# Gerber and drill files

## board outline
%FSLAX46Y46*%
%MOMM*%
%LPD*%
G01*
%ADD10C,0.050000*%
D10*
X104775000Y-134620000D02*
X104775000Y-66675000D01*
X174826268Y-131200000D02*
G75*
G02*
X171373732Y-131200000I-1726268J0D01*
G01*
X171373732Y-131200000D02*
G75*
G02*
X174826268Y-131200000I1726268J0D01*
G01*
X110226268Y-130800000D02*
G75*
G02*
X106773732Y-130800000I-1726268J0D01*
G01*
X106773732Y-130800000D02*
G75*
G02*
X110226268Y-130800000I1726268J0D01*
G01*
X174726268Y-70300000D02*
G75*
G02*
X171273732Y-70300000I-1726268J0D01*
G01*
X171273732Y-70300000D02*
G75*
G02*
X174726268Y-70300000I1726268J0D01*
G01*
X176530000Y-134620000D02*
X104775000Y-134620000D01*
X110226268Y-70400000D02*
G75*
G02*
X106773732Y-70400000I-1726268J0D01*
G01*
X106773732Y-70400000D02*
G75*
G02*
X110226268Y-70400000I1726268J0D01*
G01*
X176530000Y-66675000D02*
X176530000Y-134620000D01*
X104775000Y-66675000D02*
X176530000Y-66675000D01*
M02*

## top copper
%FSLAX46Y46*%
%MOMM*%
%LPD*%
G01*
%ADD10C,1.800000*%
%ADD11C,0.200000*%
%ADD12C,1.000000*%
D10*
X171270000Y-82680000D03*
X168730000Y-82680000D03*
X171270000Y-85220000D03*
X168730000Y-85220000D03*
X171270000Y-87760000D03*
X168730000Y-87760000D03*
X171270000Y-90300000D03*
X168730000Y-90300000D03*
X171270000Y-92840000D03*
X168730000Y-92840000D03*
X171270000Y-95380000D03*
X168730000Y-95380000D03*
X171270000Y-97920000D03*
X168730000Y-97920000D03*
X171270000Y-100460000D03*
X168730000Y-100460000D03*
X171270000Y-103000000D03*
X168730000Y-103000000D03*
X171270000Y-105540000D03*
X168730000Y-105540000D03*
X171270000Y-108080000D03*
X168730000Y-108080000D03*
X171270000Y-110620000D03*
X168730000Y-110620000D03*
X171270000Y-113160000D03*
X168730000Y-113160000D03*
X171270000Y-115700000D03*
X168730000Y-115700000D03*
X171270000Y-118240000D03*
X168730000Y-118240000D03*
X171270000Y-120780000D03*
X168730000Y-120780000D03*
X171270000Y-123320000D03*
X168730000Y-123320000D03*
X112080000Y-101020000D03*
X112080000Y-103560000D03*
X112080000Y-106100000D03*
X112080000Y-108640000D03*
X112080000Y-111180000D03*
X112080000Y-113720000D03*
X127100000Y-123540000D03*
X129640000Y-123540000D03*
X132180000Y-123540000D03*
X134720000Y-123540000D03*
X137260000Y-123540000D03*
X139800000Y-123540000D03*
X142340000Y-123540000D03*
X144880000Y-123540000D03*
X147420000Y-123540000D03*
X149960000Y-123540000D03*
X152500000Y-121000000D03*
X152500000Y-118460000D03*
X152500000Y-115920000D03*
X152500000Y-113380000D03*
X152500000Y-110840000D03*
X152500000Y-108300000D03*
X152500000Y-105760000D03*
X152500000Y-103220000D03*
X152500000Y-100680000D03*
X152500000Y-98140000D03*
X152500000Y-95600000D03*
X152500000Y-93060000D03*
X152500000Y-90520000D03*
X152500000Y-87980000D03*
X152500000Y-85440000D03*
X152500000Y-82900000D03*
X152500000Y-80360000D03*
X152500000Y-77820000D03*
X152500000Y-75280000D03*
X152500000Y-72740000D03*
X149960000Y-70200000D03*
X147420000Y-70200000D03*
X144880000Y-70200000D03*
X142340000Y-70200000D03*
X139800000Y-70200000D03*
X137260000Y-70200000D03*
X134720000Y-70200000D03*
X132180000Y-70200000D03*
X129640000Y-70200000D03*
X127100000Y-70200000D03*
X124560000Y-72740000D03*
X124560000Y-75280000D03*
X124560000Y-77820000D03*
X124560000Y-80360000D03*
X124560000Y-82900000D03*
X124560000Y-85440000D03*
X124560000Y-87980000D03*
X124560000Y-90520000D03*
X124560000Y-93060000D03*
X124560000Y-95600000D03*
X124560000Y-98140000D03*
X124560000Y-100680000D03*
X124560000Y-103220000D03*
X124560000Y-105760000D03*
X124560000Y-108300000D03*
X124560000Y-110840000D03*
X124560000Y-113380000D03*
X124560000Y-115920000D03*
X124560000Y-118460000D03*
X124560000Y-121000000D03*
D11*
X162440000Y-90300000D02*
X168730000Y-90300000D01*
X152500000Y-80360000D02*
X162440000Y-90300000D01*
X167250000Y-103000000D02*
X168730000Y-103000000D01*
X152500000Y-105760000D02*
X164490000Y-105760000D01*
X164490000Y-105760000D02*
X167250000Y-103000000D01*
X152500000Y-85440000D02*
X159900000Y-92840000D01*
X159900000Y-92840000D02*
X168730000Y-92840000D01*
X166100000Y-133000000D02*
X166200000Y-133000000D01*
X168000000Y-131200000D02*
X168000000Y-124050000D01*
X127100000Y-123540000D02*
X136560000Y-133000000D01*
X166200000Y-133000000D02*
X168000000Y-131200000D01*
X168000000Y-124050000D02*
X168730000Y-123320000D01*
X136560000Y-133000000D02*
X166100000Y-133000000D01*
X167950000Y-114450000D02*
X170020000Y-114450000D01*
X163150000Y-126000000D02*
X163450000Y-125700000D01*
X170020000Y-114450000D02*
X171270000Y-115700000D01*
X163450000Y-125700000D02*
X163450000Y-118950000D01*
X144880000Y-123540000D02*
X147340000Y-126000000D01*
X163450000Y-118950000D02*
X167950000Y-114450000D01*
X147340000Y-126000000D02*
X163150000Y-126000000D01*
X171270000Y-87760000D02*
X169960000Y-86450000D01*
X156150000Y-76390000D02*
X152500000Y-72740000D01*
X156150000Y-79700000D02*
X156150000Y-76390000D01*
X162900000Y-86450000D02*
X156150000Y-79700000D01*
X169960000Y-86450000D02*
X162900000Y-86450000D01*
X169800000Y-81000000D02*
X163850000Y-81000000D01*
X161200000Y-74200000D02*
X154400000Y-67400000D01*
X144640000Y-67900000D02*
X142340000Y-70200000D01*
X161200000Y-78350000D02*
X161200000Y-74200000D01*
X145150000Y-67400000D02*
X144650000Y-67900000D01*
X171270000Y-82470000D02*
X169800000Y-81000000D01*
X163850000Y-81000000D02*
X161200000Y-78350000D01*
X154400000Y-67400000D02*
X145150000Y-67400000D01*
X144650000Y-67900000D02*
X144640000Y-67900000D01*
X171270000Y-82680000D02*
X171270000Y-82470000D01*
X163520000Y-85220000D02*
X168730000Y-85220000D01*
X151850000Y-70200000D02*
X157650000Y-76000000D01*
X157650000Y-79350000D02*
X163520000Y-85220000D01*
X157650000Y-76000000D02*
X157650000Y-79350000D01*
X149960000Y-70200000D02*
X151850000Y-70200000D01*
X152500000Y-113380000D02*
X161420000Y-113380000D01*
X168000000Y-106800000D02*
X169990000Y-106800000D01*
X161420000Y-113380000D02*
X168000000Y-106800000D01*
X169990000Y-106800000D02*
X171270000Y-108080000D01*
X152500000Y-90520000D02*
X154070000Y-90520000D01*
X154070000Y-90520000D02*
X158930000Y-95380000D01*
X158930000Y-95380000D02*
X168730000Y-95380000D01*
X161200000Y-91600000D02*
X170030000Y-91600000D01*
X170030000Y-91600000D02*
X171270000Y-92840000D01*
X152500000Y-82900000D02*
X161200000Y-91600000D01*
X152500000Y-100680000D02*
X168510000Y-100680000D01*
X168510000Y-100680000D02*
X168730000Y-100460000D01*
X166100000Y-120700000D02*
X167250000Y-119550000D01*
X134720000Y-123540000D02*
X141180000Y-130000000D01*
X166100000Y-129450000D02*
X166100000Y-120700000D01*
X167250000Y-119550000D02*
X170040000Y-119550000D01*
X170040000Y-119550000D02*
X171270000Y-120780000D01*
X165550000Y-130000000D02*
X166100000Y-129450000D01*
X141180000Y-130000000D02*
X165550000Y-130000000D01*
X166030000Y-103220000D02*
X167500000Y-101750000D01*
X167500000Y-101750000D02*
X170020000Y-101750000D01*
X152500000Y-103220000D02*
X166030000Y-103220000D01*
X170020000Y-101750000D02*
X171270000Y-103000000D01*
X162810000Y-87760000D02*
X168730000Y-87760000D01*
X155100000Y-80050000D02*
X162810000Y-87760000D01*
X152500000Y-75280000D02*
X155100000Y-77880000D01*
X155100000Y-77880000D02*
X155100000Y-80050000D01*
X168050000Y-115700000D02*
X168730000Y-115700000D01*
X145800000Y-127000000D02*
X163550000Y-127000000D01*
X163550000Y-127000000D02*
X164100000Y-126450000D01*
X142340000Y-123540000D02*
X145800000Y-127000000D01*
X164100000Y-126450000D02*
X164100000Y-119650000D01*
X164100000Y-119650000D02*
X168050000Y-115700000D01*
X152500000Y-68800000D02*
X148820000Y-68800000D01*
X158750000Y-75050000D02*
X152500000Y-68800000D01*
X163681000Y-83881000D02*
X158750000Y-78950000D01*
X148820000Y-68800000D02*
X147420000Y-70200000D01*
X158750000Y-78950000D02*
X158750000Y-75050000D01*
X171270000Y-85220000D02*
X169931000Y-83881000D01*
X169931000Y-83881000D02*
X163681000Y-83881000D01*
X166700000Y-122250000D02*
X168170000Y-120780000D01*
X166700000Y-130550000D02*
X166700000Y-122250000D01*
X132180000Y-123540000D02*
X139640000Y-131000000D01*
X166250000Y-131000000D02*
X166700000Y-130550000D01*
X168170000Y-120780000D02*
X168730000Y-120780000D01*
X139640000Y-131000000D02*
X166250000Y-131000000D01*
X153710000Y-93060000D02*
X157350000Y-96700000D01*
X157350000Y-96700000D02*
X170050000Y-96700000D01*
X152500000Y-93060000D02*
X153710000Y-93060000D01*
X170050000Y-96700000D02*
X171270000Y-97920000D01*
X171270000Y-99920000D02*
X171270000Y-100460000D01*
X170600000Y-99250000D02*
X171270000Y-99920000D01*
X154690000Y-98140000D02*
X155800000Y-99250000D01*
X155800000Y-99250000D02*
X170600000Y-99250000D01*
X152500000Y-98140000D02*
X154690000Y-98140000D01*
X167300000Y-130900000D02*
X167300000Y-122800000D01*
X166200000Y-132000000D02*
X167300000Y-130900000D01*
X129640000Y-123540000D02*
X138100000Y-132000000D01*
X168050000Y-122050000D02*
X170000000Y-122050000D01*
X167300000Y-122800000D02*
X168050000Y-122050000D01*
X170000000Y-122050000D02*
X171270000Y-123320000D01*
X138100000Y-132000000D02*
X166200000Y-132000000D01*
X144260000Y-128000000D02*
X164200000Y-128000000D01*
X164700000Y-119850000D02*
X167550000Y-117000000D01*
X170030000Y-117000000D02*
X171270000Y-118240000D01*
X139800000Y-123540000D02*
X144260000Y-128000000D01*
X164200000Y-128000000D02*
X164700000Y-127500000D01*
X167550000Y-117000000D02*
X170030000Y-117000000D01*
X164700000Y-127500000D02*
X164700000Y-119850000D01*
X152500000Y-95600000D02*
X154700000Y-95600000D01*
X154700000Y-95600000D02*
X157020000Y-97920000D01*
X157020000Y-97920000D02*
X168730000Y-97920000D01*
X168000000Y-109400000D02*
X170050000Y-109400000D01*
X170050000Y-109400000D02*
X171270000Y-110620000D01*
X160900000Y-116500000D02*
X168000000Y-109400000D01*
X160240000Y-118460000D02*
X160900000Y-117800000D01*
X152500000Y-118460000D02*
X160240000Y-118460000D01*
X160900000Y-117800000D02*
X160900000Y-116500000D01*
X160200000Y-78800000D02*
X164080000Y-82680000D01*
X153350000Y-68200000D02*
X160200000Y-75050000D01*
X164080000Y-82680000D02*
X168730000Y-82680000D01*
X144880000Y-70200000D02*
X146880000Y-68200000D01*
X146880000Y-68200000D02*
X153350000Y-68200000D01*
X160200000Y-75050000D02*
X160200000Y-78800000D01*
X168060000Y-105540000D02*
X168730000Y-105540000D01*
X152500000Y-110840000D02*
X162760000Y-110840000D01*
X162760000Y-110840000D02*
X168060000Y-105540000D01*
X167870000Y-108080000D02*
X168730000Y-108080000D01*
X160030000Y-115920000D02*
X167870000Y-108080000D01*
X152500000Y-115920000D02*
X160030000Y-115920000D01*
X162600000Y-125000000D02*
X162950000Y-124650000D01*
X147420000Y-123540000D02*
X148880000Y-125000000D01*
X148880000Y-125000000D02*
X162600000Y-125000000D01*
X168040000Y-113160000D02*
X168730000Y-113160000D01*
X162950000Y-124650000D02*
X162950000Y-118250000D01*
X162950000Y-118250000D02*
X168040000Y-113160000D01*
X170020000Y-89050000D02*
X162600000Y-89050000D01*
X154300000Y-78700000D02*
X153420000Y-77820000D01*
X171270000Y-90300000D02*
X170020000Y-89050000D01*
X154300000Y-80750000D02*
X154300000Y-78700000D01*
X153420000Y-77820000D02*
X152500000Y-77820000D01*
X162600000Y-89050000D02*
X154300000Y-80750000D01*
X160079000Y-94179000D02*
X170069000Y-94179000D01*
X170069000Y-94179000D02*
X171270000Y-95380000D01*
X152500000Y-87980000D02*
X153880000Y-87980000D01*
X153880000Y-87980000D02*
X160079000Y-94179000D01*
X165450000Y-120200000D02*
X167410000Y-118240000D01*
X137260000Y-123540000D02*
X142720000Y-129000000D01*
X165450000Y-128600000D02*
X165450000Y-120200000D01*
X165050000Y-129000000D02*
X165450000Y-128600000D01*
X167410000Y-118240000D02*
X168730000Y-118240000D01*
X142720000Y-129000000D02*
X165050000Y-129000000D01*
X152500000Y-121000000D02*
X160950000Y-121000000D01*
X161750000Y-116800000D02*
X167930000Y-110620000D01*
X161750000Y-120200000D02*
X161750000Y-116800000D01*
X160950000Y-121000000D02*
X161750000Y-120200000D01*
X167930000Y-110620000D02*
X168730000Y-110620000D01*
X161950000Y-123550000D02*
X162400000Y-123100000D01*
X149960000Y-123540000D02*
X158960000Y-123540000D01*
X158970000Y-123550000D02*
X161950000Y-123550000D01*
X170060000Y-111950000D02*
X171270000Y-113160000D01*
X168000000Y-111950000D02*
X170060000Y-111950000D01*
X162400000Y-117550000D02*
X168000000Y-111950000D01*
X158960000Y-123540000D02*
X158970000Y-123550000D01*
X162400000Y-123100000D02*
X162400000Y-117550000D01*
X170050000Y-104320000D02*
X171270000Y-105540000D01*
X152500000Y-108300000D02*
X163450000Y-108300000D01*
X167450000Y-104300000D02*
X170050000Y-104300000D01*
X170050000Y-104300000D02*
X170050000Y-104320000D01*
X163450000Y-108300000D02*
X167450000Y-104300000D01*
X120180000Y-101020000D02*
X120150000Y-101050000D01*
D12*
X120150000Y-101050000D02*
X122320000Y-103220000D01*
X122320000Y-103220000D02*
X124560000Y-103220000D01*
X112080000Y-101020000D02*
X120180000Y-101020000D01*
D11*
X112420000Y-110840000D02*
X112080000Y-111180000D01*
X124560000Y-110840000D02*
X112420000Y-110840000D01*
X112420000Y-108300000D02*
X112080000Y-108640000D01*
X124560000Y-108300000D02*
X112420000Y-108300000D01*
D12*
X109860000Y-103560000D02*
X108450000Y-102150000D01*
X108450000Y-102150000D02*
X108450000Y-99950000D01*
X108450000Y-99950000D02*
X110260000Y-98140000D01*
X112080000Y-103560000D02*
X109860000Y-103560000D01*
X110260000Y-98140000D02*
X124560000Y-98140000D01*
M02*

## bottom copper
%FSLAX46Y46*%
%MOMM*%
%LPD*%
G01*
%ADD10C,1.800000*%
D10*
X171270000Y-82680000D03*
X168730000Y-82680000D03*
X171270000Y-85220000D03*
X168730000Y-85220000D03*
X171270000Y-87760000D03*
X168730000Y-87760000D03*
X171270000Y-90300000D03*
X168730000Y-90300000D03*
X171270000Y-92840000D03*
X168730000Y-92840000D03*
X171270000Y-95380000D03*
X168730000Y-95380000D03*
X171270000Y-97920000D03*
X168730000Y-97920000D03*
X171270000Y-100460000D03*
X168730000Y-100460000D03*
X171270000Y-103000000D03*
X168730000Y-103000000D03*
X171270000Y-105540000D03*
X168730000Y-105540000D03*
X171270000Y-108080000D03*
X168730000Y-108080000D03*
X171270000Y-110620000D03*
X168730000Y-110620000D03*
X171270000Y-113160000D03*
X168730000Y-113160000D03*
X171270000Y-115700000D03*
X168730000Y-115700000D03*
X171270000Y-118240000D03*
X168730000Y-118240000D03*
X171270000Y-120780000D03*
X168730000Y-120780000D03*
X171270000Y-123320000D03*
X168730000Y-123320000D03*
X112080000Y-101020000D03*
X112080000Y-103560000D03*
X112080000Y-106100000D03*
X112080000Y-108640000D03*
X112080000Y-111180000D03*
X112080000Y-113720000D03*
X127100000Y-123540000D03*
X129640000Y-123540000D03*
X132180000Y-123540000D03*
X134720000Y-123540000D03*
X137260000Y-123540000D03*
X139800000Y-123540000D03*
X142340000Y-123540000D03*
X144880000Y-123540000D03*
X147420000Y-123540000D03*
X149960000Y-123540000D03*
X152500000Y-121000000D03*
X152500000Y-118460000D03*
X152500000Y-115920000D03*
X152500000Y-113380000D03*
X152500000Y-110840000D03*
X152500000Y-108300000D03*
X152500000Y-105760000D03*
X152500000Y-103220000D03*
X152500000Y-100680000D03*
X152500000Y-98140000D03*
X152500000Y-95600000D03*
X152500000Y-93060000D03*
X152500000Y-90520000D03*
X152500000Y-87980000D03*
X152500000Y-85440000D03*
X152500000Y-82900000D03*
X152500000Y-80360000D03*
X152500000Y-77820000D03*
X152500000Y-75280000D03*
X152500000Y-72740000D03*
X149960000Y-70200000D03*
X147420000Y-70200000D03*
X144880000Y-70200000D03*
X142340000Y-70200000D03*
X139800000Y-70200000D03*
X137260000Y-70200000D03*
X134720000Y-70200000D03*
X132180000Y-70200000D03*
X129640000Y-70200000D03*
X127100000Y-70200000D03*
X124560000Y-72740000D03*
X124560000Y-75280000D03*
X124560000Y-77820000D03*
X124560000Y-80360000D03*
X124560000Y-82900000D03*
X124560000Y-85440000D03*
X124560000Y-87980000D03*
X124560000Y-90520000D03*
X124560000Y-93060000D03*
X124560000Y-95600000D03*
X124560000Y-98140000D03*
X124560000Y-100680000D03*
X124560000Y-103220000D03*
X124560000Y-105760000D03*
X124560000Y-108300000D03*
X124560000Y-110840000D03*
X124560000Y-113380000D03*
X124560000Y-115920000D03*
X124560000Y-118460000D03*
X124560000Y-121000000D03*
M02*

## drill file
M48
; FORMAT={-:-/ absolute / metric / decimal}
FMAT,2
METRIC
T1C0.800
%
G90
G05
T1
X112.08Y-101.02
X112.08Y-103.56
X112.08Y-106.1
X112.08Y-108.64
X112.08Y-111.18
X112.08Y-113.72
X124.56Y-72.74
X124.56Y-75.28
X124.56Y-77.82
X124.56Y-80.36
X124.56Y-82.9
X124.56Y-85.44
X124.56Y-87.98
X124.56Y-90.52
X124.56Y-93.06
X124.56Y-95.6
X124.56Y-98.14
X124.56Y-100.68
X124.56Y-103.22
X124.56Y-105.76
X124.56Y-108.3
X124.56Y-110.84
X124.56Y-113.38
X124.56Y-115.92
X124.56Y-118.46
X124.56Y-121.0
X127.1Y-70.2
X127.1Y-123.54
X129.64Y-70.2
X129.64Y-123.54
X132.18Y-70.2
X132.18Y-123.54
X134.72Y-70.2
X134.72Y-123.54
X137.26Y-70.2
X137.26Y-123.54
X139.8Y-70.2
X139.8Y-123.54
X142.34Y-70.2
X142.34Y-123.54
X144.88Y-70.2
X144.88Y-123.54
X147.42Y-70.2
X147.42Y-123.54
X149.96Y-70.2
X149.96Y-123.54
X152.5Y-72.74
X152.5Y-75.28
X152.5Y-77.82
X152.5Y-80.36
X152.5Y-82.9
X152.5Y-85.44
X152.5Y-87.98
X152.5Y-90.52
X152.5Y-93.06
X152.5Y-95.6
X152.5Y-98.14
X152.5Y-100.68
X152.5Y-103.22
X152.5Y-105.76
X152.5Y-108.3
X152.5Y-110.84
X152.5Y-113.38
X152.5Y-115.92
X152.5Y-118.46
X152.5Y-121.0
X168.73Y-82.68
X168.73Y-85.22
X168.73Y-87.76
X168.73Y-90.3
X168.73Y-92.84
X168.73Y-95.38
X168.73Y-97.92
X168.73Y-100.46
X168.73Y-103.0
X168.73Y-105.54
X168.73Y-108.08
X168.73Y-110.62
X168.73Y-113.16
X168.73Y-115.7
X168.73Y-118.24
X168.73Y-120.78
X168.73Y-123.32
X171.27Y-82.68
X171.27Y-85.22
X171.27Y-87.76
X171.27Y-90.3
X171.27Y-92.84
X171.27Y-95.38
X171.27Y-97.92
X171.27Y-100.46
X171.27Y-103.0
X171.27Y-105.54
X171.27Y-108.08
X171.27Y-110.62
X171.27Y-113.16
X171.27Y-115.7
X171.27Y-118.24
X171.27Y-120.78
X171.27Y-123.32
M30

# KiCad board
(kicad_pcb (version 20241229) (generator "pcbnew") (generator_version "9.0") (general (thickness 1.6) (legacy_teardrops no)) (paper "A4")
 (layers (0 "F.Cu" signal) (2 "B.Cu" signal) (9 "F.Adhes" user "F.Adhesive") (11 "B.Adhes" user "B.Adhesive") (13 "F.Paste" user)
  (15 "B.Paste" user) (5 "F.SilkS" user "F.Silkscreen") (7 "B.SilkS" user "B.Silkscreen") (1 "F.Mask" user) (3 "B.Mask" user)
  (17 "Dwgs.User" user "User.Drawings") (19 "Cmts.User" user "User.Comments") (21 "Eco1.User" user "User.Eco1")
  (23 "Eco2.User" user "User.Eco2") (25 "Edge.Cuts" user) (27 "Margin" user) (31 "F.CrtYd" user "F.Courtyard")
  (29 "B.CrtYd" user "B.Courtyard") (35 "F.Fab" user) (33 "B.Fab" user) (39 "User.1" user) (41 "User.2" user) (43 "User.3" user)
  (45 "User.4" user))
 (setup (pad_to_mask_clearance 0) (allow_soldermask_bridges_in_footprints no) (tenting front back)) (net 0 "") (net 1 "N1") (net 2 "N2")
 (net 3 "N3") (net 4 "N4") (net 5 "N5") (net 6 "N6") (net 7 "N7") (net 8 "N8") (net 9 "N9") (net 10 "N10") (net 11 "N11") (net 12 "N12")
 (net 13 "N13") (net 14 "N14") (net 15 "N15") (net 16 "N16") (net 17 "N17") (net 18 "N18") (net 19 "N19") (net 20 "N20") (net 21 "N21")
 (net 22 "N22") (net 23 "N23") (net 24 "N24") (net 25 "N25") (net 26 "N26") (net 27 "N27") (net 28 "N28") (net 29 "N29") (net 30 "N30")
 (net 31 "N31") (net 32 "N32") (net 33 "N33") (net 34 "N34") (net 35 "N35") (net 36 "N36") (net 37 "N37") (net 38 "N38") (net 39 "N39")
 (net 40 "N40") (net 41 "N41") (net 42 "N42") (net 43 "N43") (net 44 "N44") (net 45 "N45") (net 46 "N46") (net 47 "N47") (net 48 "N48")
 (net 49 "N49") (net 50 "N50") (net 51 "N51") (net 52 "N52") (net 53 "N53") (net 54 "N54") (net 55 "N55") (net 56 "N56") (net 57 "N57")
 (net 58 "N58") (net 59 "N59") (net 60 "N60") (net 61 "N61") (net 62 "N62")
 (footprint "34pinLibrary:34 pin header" (layer "F.Cu") (at 168.73 82.68)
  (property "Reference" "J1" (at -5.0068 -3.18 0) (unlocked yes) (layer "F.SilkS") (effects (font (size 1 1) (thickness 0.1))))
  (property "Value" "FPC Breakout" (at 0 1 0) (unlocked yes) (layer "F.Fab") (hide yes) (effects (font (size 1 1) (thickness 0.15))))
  (pad "1" thru_hole circle (at 2.54 0) (size 1.8 1.8) (drill 0.8) (layers "*.Cu" "*.Mask") (remove_unused_layers no) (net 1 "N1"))
  (pad "2" thru_hole circle (at 0 0) (size 1.8 1.8) (drill 0.8) (layers "*.Cu" "*.Mask") (remove_unused_layers no) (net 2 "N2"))
  (pad "3" thru_hole circle (at 2.54 2.54) (size 1.8 1.8) (drill 0.8) (layers "*.Cu" "*.Mask") (remove_unused_layers no) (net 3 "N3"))
  (pad "4" thru_hole circle (at 0 2.54) (size 1.8 1.8) (drill 0.8) (layers "*.Cu" "*.Mask") (remove_unused_layers no) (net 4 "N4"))
  (pad "5" thru_hole circle (at 2.54 5.08) (size 1.8 1.8) (drill 0.8) (layers "*.Cu" "*.Mask") (remove_unused_layers no) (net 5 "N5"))
  (pad "6" thru_hole circle (at 0 5.08) (size 1.8 1.8) (drill 0.8) (layers "*.Cu" "*.Mask") (remove_unused_layers no) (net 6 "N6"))
  (pad "7" thru_hole circle (at 2.54 7.62) (size 1.8 1.8) (drill 0.8) (layers "*.Cu" "*.Mask") (remove_unused_layers no) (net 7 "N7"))
  (pad "8" thru_hole circle (at 0 7.62) (size 1.8 1.8) (drill 0.8) (layers "*.Cu" "*.Mask") (remove_unused_layers no) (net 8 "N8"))
  (pad "9" thru_hole circle (at 2.54 10.16) (size 1.8 1.8) (drill 0.8) (layers "*.Cu" "*.Mask") (remove_unused_layers no) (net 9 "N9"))
  (pad "10" thru_hole circle (at 0 10.16) (size 1.8 1.8) (drill 0.8) (layers "*.Cu" "*.Mask") (remove_unused_layers no) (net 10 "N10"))
  (pad "11" thru_hole circle (at 2.54 12.7) (size 1.8 1.8) (drill 0.8) (layers "*.Cu" "*.Mask") (remove_unused_layers no) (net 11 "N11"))
  (pad "12" thru_hole circle (at 0 12.7) (size 1.8 1.8) (drill 0.8) (layers "*.Cu" "*.Mask") (remove_unused_layers no) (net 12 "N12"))
  (pad "13" thru_hole circle (at 2.54 15.24) (size 1.8 1.8) (drill 0.8) (layers "*.Cu" "*.Mask") (remove_unused_layers no) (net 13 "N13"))
  (pad "14" thru_hole circle (at 0 15.24) (size 1.8 1.8) (drill 0.8) (layers "*.Cu" "*.Mask") (remove_unused_layers no) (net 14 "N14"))
  (pad "15" thru_hole circle (at 2.54 17.78) (size 1.8 1.8) (drill 0.8) (layers "*.Cu" "*.Mask") (remove_unused_layers no) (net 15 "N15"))
  (pad "16" thru_hole circle (at 0 17.78) (size 1.8 1.8) (drill 0.8) (layers "*.Cu" "*.Mask") (remove_unused_layers no) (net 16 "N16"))
  (pad "17" thru_hole circle (at 2.54 20.32) (size 1.8 1.8) (drill 0.8) (layers "*.Cu" "*.Mask") (remove_unused_layers no) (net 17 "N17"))
  (pad "18" thru_hole circle (at 0 20.32) (size 1.8 1.8) (drill 0.8) (layers "*.Cu" "*.Mask") (remove_unused_layers no) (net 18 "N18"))
  (pad "19" thru_hole circle (at 2.54 22.86) (size 1.8 1.8) (drill 0.8) (layers "*.Cu" "*.Mask") (remove_unused_layers no) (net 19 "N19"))
  (pad "20" thru_hole circle (at 0 22.86) (size 1.8 1.8) (drill 0.8) (layers "*.Cu" "*.Mask") (remove_unused_layers no) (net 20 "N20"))
  (pad "21" thru_hole circle (at 2.54 25.4) (size 1.8 1.8) (drill 0.8) (layers "*.Cu" "*.Mask") (remove_unused_layers no) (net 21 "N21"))
  (pad "22" thru_hole circle (at 0 25.4) (size 1.8 1.8) (drill 0.8) (layers "*.Cu" "*.Mask") (remove_unused_layers no) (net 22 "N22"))
  (pad "23" thru_hole circle (at 2.54 27.94) (size 1.8 1.8) (drill 0.8) (layers "*.Cu" "*.Mask") (remove_unused_layers no) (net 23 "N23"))
  (pad "24" thru_hole circle (at 0 27.94) (size 1.8 1.8) (drill 0.8) (layers "*.Cu" "*.Mask") (remove_unused_layers no) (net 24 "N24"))
  (pad "25" thru_hole circle (at 2.54 30.48) (size 1.8 1.8) (drill 0.8) (layers "*.Cu" "*.Mask") (remove_unused_layers no) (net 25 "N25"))
  (pad "26" thru_hole circle (at 0 30.48) (size 1.8 1.8) (drill 0.8) (layers "*.Cu" "*.Mask") (remove_unused_layers no) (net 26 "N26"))
  (pad "27" thru_hole circle (at 2.54 33.02) (size 1.8 1.8) (drill 0.8) (layers "*.Cu" "*.Mask") (remove_unused_layers no) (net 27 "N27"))
  (pad "28" thru_hole circle (at 0 33.02) (size 1.8 1.8) (drill 0.8) (layers "*.Cu" "*.Mask") (remove_unused_layers no) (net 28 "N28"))
  (pad "29" thru_hole circle (at 2.54 35.56) (size 1.8 1.8) (drill 0.8) (layers "*.Cu" "*.Mask") (remove_unused_layers no) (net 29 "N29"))
  (pad "30" thru_hole circle (at 0 35.56) (size 1.8 1.8) (drill 0.8) (layers "*.Cu" "*.Mask") (remove_unused_layers no) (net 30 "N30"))
  (pad "31" thru_hole circle (at 2.54 38.1) (size 1.8 1.8) (drill 0.8) (layers "*.Cu" "*.Mask") (remove_unused_layers no) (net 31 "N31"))
  (pad "32" thru_hole circle (at 0 38.1) (size 1.8 1.8) (drill 0.8) (layers "*.Cu" "*.Mask") (remove_unused_layers no) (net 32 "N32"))
  (pad "33" thru_hole circle (at 2.54 40.64) (size 1.8 1.8) (drill 0.8) (layers "*.Cu" "*.Mask") (remove_unused_layers no) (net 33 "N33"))
  (pad "34" thru_hole circle (at 0 40.64) (size 1.8 1.8) (drill 0.8) (layers "*.Cu" "*.Mask") (remove_unused_layers no) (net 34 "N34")))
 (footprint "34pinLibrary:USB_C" (layer "F.Cu") (at 112.08 93.4)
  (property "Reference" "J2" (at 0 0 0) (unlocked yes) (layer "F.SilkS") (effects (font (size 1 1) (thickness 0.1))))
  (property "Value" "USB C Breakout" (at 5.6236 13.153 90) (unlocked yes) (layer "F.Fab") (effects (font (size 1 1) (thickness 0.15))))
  (pad "1" thru_hole circle (at 0 7.62) (size 1.8 1.8) (drill 0.8) (layers "*.Cu" "*.Mask") (remove_unused_layers no) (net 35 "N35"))
  (pad "2" thru_hole circle (at 0 10.16) (size 1.8 1.8) (drill 0.8) (layers "*.Cu" "*.Mask") (remove_unused_layers no) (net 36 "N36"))
  (pad "3" thru_hole circle (at 0 12.7) (size 1.8 1.8) (drill 0.8) (layers "*.Cu" "*.Mask") (remove_unused_layers no) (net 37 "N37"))
  (pad "4" thru_hole circle (at 0 15.24) (size 1.8 1.8) (drill 0.8) (layers "*.Cu" "*.Mask") (remove_unused_layers no) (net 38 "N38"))
  (pad "5" thru_hole circle (at 0 17.78) (size 1.8 1.8) (drill 0.8) (layers "*.Cu" "*.Mask") (remove_unused_layers no) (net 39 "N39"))
  (pad "6" thru_hole circle (at 0 20.32) (size 1.8 1.8) (drill 0.8) (layers "*.Cu" "*.Mask") (remove_unused_layers no) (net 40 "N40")))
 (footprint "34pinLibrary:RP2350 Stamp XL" (layer "F.Cu") (at 137.26 67.66)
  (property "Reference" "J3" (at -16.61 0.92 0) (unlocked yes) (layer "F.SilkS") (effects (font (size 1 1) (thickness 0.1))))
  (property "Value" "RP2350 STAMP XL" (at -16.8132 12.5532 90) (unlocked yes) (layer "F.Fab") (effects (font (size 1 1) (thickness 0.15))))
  (pad "1" thru_hole circle (at -10.16 55.88) (size 1.8 1.8) (drill 0.8) (layers "*.Cu" "*.Mask") (remove_unused_layers no) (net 34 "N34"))
  (pad "2" thru_hole circle (at -7.62 55.88) (size 1.8 1.8) (drill 0.8) (layers "*.Cu" "*.Mask") (remove_unused_layers no) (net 33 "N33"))
  (pad "3" thru_hole circle (at -5.08 55.88) (size 1.8 1.8) (drill 0.8) (layers "*.Cu" "*.Mask") (remove_unused_layers no) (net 32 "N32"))
  (pad "4" thru_hole circle (at -2.54 55.88) (size 1.8 1.8) (drill 0.8) (layers "*.Cu" "*.Mask") (remove_unused_layers no) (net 31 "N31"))
  (pad "5" thru_hole circle (at 0 55.88) (size 1.8 1.8) (drill 0.8) (layers "*.Cu" "*.Mask") (remove_unused_layers no) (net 30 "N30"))
  (pad "6" thru_hole circle (at 2.54 55.88) (size 1.8 1.8) (drill 0.8) (layers "*.Cu" "*.Mask") (remove_unused_layers no) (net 29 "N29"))
  (pad "7" thru_hole circle (at 5.08 55.88) (size 1.8 1.8) (drill 0.8) (layers "*.Cu" "*.Mask") (remove_unused_layers no) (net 28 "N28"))
  (pad "8" thru_hole circle (at 7.62 55.88) (size 1.8 1.8) (drill 0.8) (layers "*.Cu" "*.Mask") (remove_unused_layers no) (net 27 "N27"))
  (pad "9" thru_hole circle (at 10.16 55.88) (size 1.8 1.8) (drill 0.8) (layers "*.Cu" "*.Mask") (remove_unused_layers no) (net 26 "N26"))
  (pad "10" thru_hole circle (at 12.7 55.88) (size 1.8 1.8) (drill 0.8) (layers "*.Cu" "*.Mask") (remove_unused_layers no) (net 25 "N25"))
  (pad "11" thru_hole circle (at 15.24 53.34) (size 1.8 1.8) (drill 0.8) (layers "*.Cu" "*.Mask") (remove_unused_layers no) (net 24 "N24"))
  (pad "12" thru_hole circle (at 15.24 50.8) (size 1.8 1.8) (drill 0.8) (layers "*.Cu" "*.Mask") (remove_unused_layers no) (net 23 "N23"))
  (pad "13" thru_hole circle (at 15.24 48.26) (size 1.8 1.8) (drill 0.8) (layers "*.Cu" "*.Mask") (remove_unused_layers no) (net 22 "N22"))
  (pad "14" thru_hole circle (at 15.24 45.72) (size 1.8 1.8) (drill 0.8) (layers "*.Cu" "*.Mask") (remove_unused_layers no) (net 21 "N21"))
  (pad "15" thru_hole circle (at 15.24 43.18) (size 1.8 1.8) (drill 0.8) (layers "*.Cu" "*.Mask") (remove_unused_layers no) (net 20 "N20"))
  (pad "16" thru_hole circle (at 15.24 40.64) (size 1.8 1.8) (drill 0.8) (layers "*.Cu" "*.Mask") (remove_unused_layers no) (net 19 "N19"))
  (pad "17" thru_hole circle (at 15.24 38.1) (size 1.8 1.8) (drill 0.8) (layers "*.Cu" "*.Mask") (remove_unused_layers no) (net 18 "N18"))
  (pad "18" thru_hole circle (at 15.24 35.56) (size 1.8 1.8) (drill 0.8) (layers "*.Cu" "*.Mask") (remove_unused_layers no) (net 17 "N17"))
  (pad "19" thru_hole circle (at 15.24 33.02) (size 1.8 1.8) (drill 0.8) (layers "*.Cu" "*.Mask") (remove_unused_layers no) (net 16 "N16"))
  (pad "20" thru_hole circle (at 15.24 30.48) (size 1.8 1.8) (drill 0.8) (layers "*.Cu" "*.Mask") (remove_unused_layers no) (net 15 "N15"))
  (pad "21" thru_hole circle (at 15.24 27.94) (size 1.8 1.8) (drill 0.8) (layers "*.Cu" "*.Mask") (remove_unused_layers no) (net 14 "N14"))
  (pad "22" thru_hole circle (at 15.24 25.4) (size 1.8 1.8) (drill 0.8) (layers "*.Cu" "*.Mask") (remove_unused_layers no) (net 13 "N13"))
  (pad "23" thru_hole circle (at 15.24 22.86) (size 1.8 1.8) (drill 0.8) (layers "*.Cu" "*.Mask") (remove_unused_layers no) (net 12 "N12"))
  (pad "24" thru_hole circle (at 15.24 20.32) (size 1.8 1.8) (drill 0.8) (layers "*.Cu" "*.Mask") (remove_unused_layers no) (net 11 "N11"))
  (pad "25" thru_hole circle (at 15.24 17.78) (size 1.8 1.8) (drill 0.8) (layers "*.Cu" "*.Mask") (remove_unused_layers no) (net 10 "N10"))
  (pad "26" thru_hole circle (at 15.24 15.24) (size 1.8 1.8) (drill 0.8) (layers "*.Cu" "*.Mask") (remove_unused_layers no) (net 9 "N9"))
  (pad "27" thru_hole circle (at 15.24 12.7) (size 1.8 1.8) (drill 0.8) (layers "*.Cu" "*.Mask") (remove_unused_layers no) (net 8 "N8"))
  (pad "28" thru_hole circle (at 15.24 10.16) (size 1.8 1.8) (drill 0.8) (layers "*.Cu" "*.Mask") (remove_unused_layers no) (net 7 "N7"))
  (pad "29" thru_hole circle (at 15.24 7.62) (size 1.8 1.8) (drill 0.8) (layers "*.Cu" "*.Mask") (remove_unused_layers no) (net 6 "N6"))
  (pad "30" thru_hole circle (at 15.24 5.08) (size 1.8 1.8) (drill 0.8) (layers "*.Cu" "*.Mask") (remove_unused_layers no) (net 5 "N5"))
  (pad "31" thru_hole circle (at 12.7 2.54) (size 1.8 1.8) (drill 0.8) (layers "*.Cu" "*.Mask") (remove_unused_layers no) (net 4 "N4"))
  (pad "32" thru_hole circle (at 10.16 2.54) (size 1.8 1.8) (drill 0.8) (layers "*.Cu" "*.Mask") (remove_unused_layers no) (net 3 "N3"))
  (pad "33" thru_hole circle (at 7.62 2.54) (size 1.8 1.8) (drill 0.8) (layers "*.Cu" "*.Mask") (remove_unused_layers no) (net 2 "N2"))
  (pad "34" thru_hole circle (at 5.08 2.54) (size 1.8 1.8) (drill 0.8) (layers "*.Cu" "*.Mask") (remove_unused_layers no) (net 1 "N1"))
  (pad "35" thru_hole circle (at 2.54 2.54) (size 1.8 1.8) (drill 0.8) (layers "*.Cu" "*.Mask") (remove_unused_layers no) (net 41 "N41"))
  (pad "36" thru_hole circle (at 0 2.54) (size 1.8 1.8) (drill 0.8) (layers "*.Cu" "*.Mask") (remove_unused_layers no) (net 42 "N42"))
  (pad "37" thru_hole circle (at -2.54 2.54) (size 1.8 1.8) (drill 0.8) (layers "*.Cu" "*.Mask") (remove_unused_layers no) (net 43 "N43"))
  (pad "38" thru_hole circle (at -5.08 2.54) (size 1.8 1.8) (drill 0.8) (layers "*.Cu" "*.Mask") (remove_unused_layers no) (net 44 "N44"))
  (pad "39" thru_hole circle (at -7.62 2.54) (size 1.8 1.8) (drill 0.8) (layers "*.Cu" "*.Mask") (remove_unused_layers no) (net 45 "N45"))
  (pad "40" thru_hole circle (at -10.16 2.54) (size 1.8 1.8) (drill 0.8) (layers "*.Cu" "*.Mask") (remove_unused_layers no) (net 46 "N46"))
  (pad "41" thru_hole circle (at -12.7 5.08) (size 1.8 1.8) (drill 0.8) (layers "*.Cu" "*.Mask") (remove_unused_layers no) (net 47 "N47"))
  (pad "42" thru_hole circle (at -12.7 7.62) (size 1.8 1.8) (drill 0.8) (layers "*.Cu" "*.Mask") (remove_unused_layers no) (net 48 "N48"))
  (pad "43" thru_hole circle (at -12.7 10.16) (size 1.8 1.8) (drill 0.8) (layers "*.Cu" "*.Mask") (remove_unused_layers no) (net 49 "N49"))
  (pad "44" thru_hole circle (at -12.7 12.7) (size 1.8 1.8) (drill 0.8) (layers "*.Cu" "*.Mask") (remove_unused_layers no) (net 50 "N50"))
  (pad "45" thru_hole circle (at -12.7 15.24) (size 1.8 1.8) (drill 0.8) (layers "*.Cu" "*.Mask") (remove_unused_layers no) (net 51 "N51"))
  (pad "46" thru_hole circle (at -12.7 17.78) (size 1.8 1.8) (drill 0.8) (layers "*.Cu" "*.Mask") (remove_unused_layers no) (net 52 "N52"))
  (pad "47" thru_hole circle (at -12.7 20.32) (size 1.8 1.8) (drill 0.8) (layers "*.Cu" "*.Mask") (remove_unused_layers no) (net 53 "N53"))
  (pad "48" thru_hole circle (at -12.7 22.86) (size 1.8 1.8) (drill 0.8) (layers "*.Cu" "*.Mask") (remove_unused_layers no) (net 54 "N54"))
  (pad "49" thru_hole circle (at -12.7 25.4) (size 1.8 1.8) (drill 0.8) (layers "*.Cu" "*.Mask") (remove_unused_layers no) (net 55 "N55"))
  (pad "50" thru_hole circle (at -12.7 27.94) (size 1.8 1.8) (drill 0.8) (layers "*.Cu" "*.Mask") (remove_unused_layers no) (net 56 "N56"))
  (pad "51" thru_hole circle (at -12.7 30.48) (size 1.8 1.8) (drill 0.8) (layers "*.Cu" "*.Mask") (remove_unused_layers no) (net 36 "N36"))
  (pad "52" thru_hole circle (at -12.7 33.02) (size 1.8 1.8) (drill 0.8) (layers "*.Cu" "*.Mask") (remove_unused_layers no) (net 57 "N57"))
  (pad "53" thru_hole circle (at -12.7 35.56) (size 1.8 1.8) (drill 0.8) (layers "*.Cu" "*.Mask") (remove_unused_layers no) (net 35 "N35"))
  (pad "54" thru_hole circle (at -12.7 38.1) (size 1.8 1.8) (drill 0.8) (layers "*.Cu" "*.Mask") (remove_unused_layers no) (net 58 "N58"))
  (pad "55" thru_hole circle (at -12.7 40.64) (size 1.8 1.8) (drill 0.8) (layers "*.Cu" "*.Mask") (remove_unused_layers no) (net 38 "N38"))
  (pad "56" thru_hole circle (at -12.7 43.18) (size 1.8 1.8) (drill 0.8) (layers "*.Cu" "*.Mask") (remove_unused_layers no) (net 39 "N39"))
  (pad "57" thru_hole circle (at -12.7 45.72) (size 1.8 1.8) (drill 0.8) (layers "*.Cu" "*.Mask") (remove_unused_layers no) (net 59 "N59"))
  (pad "58" thru_hole circle (at -12.7 48.26) (size 1.8 1.8) (drill 0.8) (layers "*.Cu" "*.Mask") (remove_unused_layers no) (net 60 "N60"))
  (pad "59" thru_hole circle (at -12.7 50.8) (size 1.8 1.8) (drill 0.8) (layers "*.Cu" "*.Mask") (remove_unused_layers no) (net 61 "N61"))
  (pad "60" thru_hole circle (at -12.7 53.34) (size 1.8 1.8) (drill 0.8) (layers "*.Cu" "*.Mask") (remove_unused_layers no) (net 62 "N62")))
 (gr_line (start 104.775 134.62) (end 104.775 66.675) (stroke (width 0.05) (type default)) (layer "Edge.Cuts"))
 (gr_circle (center 173.1 131.2) (end 173.4 129.5) (stroke (width 0.05) (type default)) (fill no) (layer "Edge.Cuts"))
 (gr_circle (center 108.5 130.8) (end 108.8 129.1) (stroke (width 0.05) (type default)) (fill no) (layer "Edge.Cuts"))
 (gr_circle (center 173 70.3) (end 173.3 68.6) (stroke (width 0.05) (type default)) (fill no) (layer "Edge.Cuts"))
 (gr_line (start 176.53 134.62) (end 104.775 134.62) (stroke (width 0.05) (type default)) (layer "Edge.Cuts"))
 (gr_circle (center 108.5 70.4) (end 108.8 68.7) (stroke (width 0.05) (type default)) (fill no) (layer "Edge.Cuts"))
 (gr_line (start 176.53 66.675) (end 176.53 134.62) (stroke (width 0.05) (type default)) (layer "Edge.Cuts"))
 (gr_line (start 104.775 66.675) (end 176.53 66.675) (stroke (width 0.05) (type default)) (layer "Edge.Cuts"))
 (segment (start 162.44 90.3) (end 168.73 90.3) (width 0.2) (layer "F.Cu") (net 8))
 (segment (start 152.5 80.36) (end 162.44 90.3) (width 0.2) (layer "F.Cu") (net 8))
 (segment (start 167.25 103) (end 168.73 103) (width 0.2) (layer "F.Cu") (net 18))
 (segment (start 152.5 105.76) (end 164.49 105.76) (width 0.2) (layer "F.Cu") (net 18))
 (segment (start 164.49 105.76) (end 167.25 103) (width 0.2) (layer "F.Cu") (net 18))
 (segment (start 152.5 85.44) (end 159.9 92.84) (width 0.2) (layer "F.Cu") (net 10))
 (segment (start 159.9 92.84) (end 168.73 92.84) (width 0.2) (layer "F.Cu") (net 10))
 (segment (start 166.1 133) (end 166.2 133) (width 0.2) (layer "F.Cu") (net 34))
 (segment (start 168 131.2) (end 168 124.05) (width 0.2) (layer "F.Cu") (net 34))
 (segment (start 127.1 123.54) (end 136.56 133) (width 0.2) (layer "F.Cu") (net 34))
 (segment (start 166.2 133) (end 168 131.2) (width 0.2) (layer "F.Cu") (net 34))
 (segment (start 168 124.05) (end 168.73 123.32) (width 0.2) (layer "F.Cu") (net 34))
 (segment (start 136.56 133) (end 166.1 133) (width 0.2) (layer "F.Cu") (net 34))
 (segment (start 167.95 114.45) (end 170.02 114.45) (width 0.2) (layer "F.Cu") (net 27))
 (segment (start 163.15 126) (end 163.45 125.7) (width 0.2) (layer "F.Cu") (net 27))
 (segment (start 170.02 114.45) (end 171.27 115.7) (width 0.2) (layer "F.Cu") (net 27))
 (segment (start 163.45 125.7) (end 163.45 118.95) (width 0.2) (layer "F.Cu") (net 27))
 (segment (start 144.88 123.54) (end 147.34 126) (width 0.2) (layer "F.Cu") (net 27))
 (segment (start 163.45 118.95) (end 167.95 114.45) (width 0.2) (layer "F.Cu") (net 27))
 (segment (start 147.34 126) (end 163.15 126) (width 0.2) (layer "F.Cu") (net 27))
 (segment (start 171.27 87.76) (end 169.96 86.45) (width 0.2) (layer "F.Cu") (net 5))
 (segment (start 156.15 76.39) (end 152.5 72.74) (width 0.2) (layer "F.Cu") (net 5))
 (segment (start 156.15 79.7) (end 156.15 76.39) (width 0.2) (layer "F.Cu") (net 5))
 (segment (start 162.9 86.45) (end 156.15 79.7) (width 0.2) (layer "F.Cu") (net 5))
 (segment (start 169.96 86.45) (end 162.9 86.45) (width 0.2) (layer "F.Cu") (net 5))
 (segment (start 169.8 81) (end 163.85 81) (width 0.2) (layer "F.Cu") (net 1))
 (segment (start 161.2 74.2) (end 154.4 67.4) (width 0.2) (layer "F.Cu") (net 1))
 (segment (start 144.64 67.9) (end 142.34 70.2) (width 0.2) (layer "F.Cu") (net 1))
 (segment (start 161.2 78.35) (end 161.2 74.2) (width 0.2) (layer "F.Cu") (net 1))
 (segment (start 145.15 67.4) (end 144.65 67.9) (width 0.2) (layer "F.Cu") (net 1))
 (segment (start 171.27 82.47) (end 169.8 81) (width 0.2) (layer "F.Cu") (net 1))
 (segment (start 163.85 81) (end 161.2 78.35) (width 0.2) (layer "F.Cu") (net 1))
 (segment (start 154.4 67.4) (end 145.15 67.4) (width 0.2) (layer "F.Cu") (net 1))
 (segment (start 144.65 67.9) (end 144.64 67.9) (width 0.2) (layer "F.Cu") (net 1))
 (segment (start 171.27 82.68) (end 171.27 82.47) (width 0.2) (layer "F.Cu") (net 1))
 (segment (start 163.52 85.22) (end 168.73 85.22) (width 0.2) (layer "F.Cu") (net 4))
 (segment (start 151.85 70.2) (end 157.65 76) (width 0.2) (layer "F.Cu") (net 4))
 (segment (start 157.65 79.35) (end 163.52 85.22) (width 0.2) (layer "F.Cu") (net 4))
 (segment (start 157.65 76) (end 157.65 79.35) (width 0.2) (layer "F.Cu") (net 4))
 (segment (start 149.96 70.2) (end 151.85 70.2) (width 0.2) (layer "F.Cu") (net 4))
 (segment (start 152.5 113.38) (end 161.42 113.38) (width 0.2) (layer "F.Cu") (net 21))
 (segment (start 168 106.8) (end 169.99 106.8) (width 0.2) (layer "F.Cu") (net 21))
 (segment (start 161.42 113.38) (end 168 106.8) (width 0.2) (layer "F.Cu") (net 21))
 (segment (start 169.99 106.8) (end 171.27 108.08) (width 0.2) (layer "F.Cu") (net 21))
 (segment (start 152.5 90.52) (end 154.07 90.52) (width 0.2) (layer "F.Cu") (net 12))
 (segment (start 154.07 90.52) (end 158.93 95.38) (width 0.2) (layer "F.Cu") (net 12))
 (segment (start 158.93 95.38) (end 168.73 95.38) (width 0.2) (layer "F.Cu") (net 12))
 (segment (start 161.2 91.6) (end 170.03 91.6) (width 0.2) (layer "F.Cu") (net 9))
 (segment (start 170.03 91.6) (end 171.27 92.84) (width 0.2) (layer "F.Cu") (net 9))
 (segment (start 152.5 82.9) (end 161.2 91.6) (width 0.2) (layer "F.Cu") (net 9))
 (segment (start 152.5 100.68) (end 168.51 100.68) (width 0.2) (layer "F.Cu") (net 16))
 (segment (start 168.51 100.68) (end 168.73 100.46) (width 0.2) (layer "F.Cu") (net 16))
 (segment (start 166.1 120.7) (end 167.25 119.55) (width 0.2) (layer "F.Cu") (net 31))
 (segment (start 134.72 123.54) (end 141.18 130) (width 0.2) (layer "F.Cu") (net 31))
 (segment (start 166.1 129.45) (end 166.1 120.7) (width 0.2) (layer "F.Cu") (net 31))
 (segment (start 167.25 119.55) (end 170.04 119.55) (width 0.2) (layer "F.Cu") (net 31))
 (segment (start 170.04 119.55) (end 171.27 120.78) (width 0.2) (layer "F.Cu") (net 31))
 (segment (start 165.55 130) (end 166.1 129.45) (width 0.2) (layer "F.Cu") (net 31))
 (segment (start 141.18 130) (end 165.55 130) (width 0.2) (layer "F.Cu") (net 31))
 (segment (start 166.03 103.22) (end 167.5 101.75) (width 0.2) (layer "F.Cu") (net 17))
 (segment (start 167.5 101.75) (end 170.02 101.75) (width 0.2) (layer "F.Cu") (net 17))
 (segment (start 152.5 103.22) (end 166.03 103.22) (width 0.2) (layer "F.Cu") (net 17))
 (segment (start 170.02 101.75) (end 171.27 103) (width 0.2) (layer "F.Cu") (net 17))
 (segment (start 162.81 87.76) (end 168.73 87.76) (width 0.2) (layer "F.Cu") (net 6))
 (segment (start 155.1 80.05) (end 162.81 87.76) (width 0.2) (layer "F.Cu") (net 6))
 (segment (start 152.5 75.28) (end 155.1 77.88) (width 0.2) (layer "F.Cu") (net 6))
 (segment (start 155.1 77.88) (end 155.1 80.05) (width 0.2) (layer "F.Cu") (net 6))
 (segment (start 168.05 115.7) (end 168.73 115.7) (width 0.2) (layer "F.Cu") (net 28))
 (segment (start 145.8 127) (end 163.55 127) (width 0.2) (layer "F.Cu") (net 28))
 (segment (start 163.55 127) (end 164.1 126.45) (width 0.2) (layer "F.Cu") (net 28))
 (segment (start 142.34 123.54) (end 145.8 127) (width 0.2) (layer "F.Cu") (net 28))
 (segment (start 164.1 126.45) (end 164.1 119.65) (width 0.2) (layer "F.Cu") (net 28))
 (segment (start 164.1 119.65) (end 168.05 115.7) (width 0.2) (layer "F.Cu") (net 28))
 (segment (start 152.5 68.8) (end 148.82 68.8) (width 0.2) (layer "F.Cu") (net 3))
 (segment (start 158.75 75.05) (end 152.5 68.8) (width 0.2) (layer "F.Cu") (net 3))
 (segment (start 163.681 83.881) (end 158.75 78.95) (width 0.2) (layer "F.Cu") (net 3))
 (segment (start 148.82 68.8) (end 147.42 70.2) (width 0.2) (layer "F.Cu") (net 3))
 (segment (start 158.75 78.95) (end 158.75 75.05) (width 0.2) (layer "F.Cu") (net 3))
 (segment (start 171.27 85.22) (end 169.931 83.881) (width 0.2) (layer "F.Cu") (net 3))
 (segment (start 169.931 83.881) (end 163.681 83.881) (width 0.2) (layer "F.Cu") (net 3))
 (segment (start 166.7 122.25) (end 168.17 120.78) (width 0.2) (layer "F.Cu") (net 32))
 (segment (start 166.7 130.55) (end 166.7 122.25) (width 0.2) (layer "F.Cu") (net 32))
 (segment (start 132.18 123.54) (end 139.64 131) (width 0.2) (layer "F.Cu") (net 32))
 (segment (start 166.25 131) (end 166.7 130.55) (width 0.2) (layer "F.Cu") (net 32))
 (segment (start 168.17 120.78) (end 168.73 120.78) (width 0.2) (layer "F.Cu") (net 32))
 (segment (start 139.64 131) (end 166.25 131) (width 0.2) (layer "F.Cu") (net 32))
 (segment (start 153.71 93.06) (end 157.35 96.7) (width 0.2) (layer "F.Cu") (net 13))
 (segment (start 157.35 96.7) (end 170.05 96.7) (width 0.2) (layer "F.Cu") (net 13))
 (segment (start 152.5 93.06) (end 153.71 93.06) (width 0.2) (layer "F.Cu") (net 13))
 (segment (start 170.05 96.7) (end 171.27 97.92) (width 0.2) (layer "F.Cu") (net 13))
 (segment (start 171.27 99.92) (end 171.27 100.46) (width 0.2) (layer "F.Cu") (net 15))
 (segment (start 170.6 99.25) (end 171.27 99.92) (width 0.2) (layer "F.Cu") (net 15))
 (segment (start 154.69 98.14) (end 155.8 99.25) (width 0.2) (layer "F.Cu") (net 15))
 (segment (start 155.8 99.25) (end 170.6 99.25) (width 0.2) (layer "F.Cu") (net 15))
 (segment (start 152.5 98.14) (end 154.69 98.14) (width 0.2) (layer "F.Cu") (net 15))
 (segment (start 167.3 130.9) (end 167.3 122.8) (width 0.2) (layer "F.Cu") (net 33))
 (segment (start 166.2 132) (end 167.3 130.9) (width 0.2) (layer "F.Cu") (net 33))
 (segment (start 129.64 123.54) (end 138.1 132) (width 0.2) (layer "F.Cu") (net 33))
 (segment (start 168.05 122.05) (end 170 122.05) (width 0.2) (layer "F.Cu") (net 33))
 (segment (start 167.3 122.8) (end 168.05 122.05) (width 0.2) (layer "F.Cu") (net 33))
 (segment (start 170 122.05) (end 171.27 123.32) (width 0.2) (layer "F.Cu") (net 33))
 (segment (start 138.1 132) (end 166.2 132) (width 0.2) (layer "F.Cu") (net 33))
 (segment (start 144.26 128) (end 164.2 128) (width 0.2) (layer "F.Cu") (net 29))
 (segment (start 164.7 119.85) (end 167.55 117) (width 0.2) (layer "F.Cu") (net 29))
 (segment (start 170.03 117) (end 171.27 118.24) (width 0.2) (layer "F.Cu") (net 29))
 (segment (start 139.8 123.54) (end 144.26 128) (width 0.2) (layer "F.Cu") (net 29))
 (segment (start 164.2 128) (end 164.7 127.5) (width 0.2) (layer "F.Cu") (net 29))
 (segment (start 167.55 117) (end 170.03 117) (width 0.2) (layer "F.Cu") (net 29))
 (segment (start 164.7 127.5) (end 164.7 119.85) (width 0.2) (layer "F.Cu") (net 29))
 (segment (start 152.5 95.6) (end 154.7 95.6) (width 0.2) (layer "F.Cu") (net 14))
 (segment (start 154.7 95.6) (end 157.02 97.92) (width 0.2) (layer "F.Cu") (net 14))
 (segment (start 157.02 97.92) (end 168.73 97.92) (width 0.2) (layer "F.Cu") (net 14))
 (segment (start 168 109.4) (end 170.05 109.4) (width 0.2) (layer "F.Cu") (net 23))
 (segment (start 170.05 109.4) (end 171.27 110.62) (width 0.2) (layer "F.Cu") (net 23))
 (segment (start 160.9 116.5) (end 168 109.4) (width 0.2) (layer "F.Cu") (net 23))
 (segment (start 160.24 118.46) (end 160.9 117.8) (width 0.2) (layer "F.Cu") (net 23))
 (segment (start 152.5 118.46) (end 160.24 118.46) (width 0.2) (layer "F.Cu") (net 23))
 (segment (start 160.9 117.8) (end 160.9 116.5) (width 0.2) (layer "F.Cu") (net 23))
 (segment (start 160.2 78.8) (end 164.08 82.68) (width 0.2) (layer "F.Cu") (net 2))
 (segment (start 153.35 68.2) (end 160.2 75.05) (width 0.2) (layer "F.Cu") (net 2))
 (segment (start 164.08 82.68) (end 168.73 82.68) (width 0.2) (layer "F.Cu") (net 2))
 (segment (start 144.88 70.2) (end 146.88 68.2) (width 0.2) (layer "F.Cu") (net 2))
 (segment (start 146.88 68.2) (end 153.35 68.2) (width 0.2) (layer "F.Cu") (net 2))
 (segment (start 160.2 75.05) (end 160.2 78.8) (width 0.2) (layer "F.Cu") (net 2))
 (segment (start 168.06 105.54) (end 168.73 105.54) (width 0.2) (layer "F.Cu") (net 20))
 (segment (start 152.5 110.84) (end 162.76 110.84) (width 0.2) (layer "F.Cu") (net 20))
 (segment (start 162.76 110.84) (end 168.06 105.54) (width 0.2) (layer "F.Cu") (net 20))
 (segment (start 167.87 108.08) (end 168.73 108.08) (width 0.2) (layer "F.Cu") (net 22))
 (segment (start 160.03 115.92) (end 167.87 108.08) (width 0.2) (layer "F.Cu") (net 22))
 (segment (start 152.5 115.92) (end 160.03 115.92) (width 0.2) (layer "F.Cu") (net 22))
 (segment (start 162.6 125) (end 162.95 124.65) (width 0.2) (layer "F.Cu") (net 26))
 (segment (start 147.42 123.54) (end 148.88 125) (width 0.2) (layer "F.Cu") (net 26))
 (segment (start 148.88 125) (end 162.6 125) (width 0.2) (layer "F.Cu") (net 26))
 (segment (start 168.04 113.16) (end 168.73 113.16) (width 0.2) (layer "F.Cu") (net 26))
 (segment (start 162.95 124.65) (end 162.95 118.25) (width 0.2) (layer "F.Cu") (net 26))
 (segment (start 162.95 118.25) (end 168.04 113.16) (width 0.2) (layer "F.Cu") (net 26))
 (segment (start 170.02 89.05) (end 162.6 89.05) (width 0.2) (layer "F.Cu") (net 7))
 (segment (start 154.3 78.7) (end 153.42 77.82) (width 0.2) (layer "F.Cu") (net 7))
 (segment (start 171.27 90.3) (end 170.02 89.05) (width 0.2) (layer "F.Cu") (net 7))
 (segment (start 154.3 80.75) (end 154.3 78.7) (width 0.2) (layer "F.Cu") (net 7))
 (segment (start 153.42 77.82) (end 152.5 77.82) (width 0.2) (layer "F.Cu") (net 7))
 (segment (start 162.6 89.05) (end 154.3 80.75) (width 0.2) (layer "F.Cu") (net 7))
 (segment (start 160.079 94.179) (end 170.069 94.179) (width 0.2) (layer "F.Cu") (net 11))
 (segment (start 170.069 94.179) (end 171.27 95.38) (width 0.2) (layer "F.Cu") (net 11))
 (segment (start 152.5 87.98) (end 153.88 87.98) (width 0.2) (layer "F.Cu") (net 11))
 (segment (start 153.88 87.98) (end 160.079 94.179) (width 0.2) (layer "F.Cu") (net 11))
 (segment (start 165.45 120.2) (end 167.41 118.24) (width 0.2) (layer "F.Cu") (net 30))
 (segment (start 137.26 123.54) (end 142.72 129) (width 0.2) (layer "F.Cu") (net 30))
 (segment (start 165.45 128.6) (end 165.45 120.2) (width 0.2) (layer "F.Cu") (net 30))
 (segment (start 165.05 129) (end 165.45 128.6) (width 0.2) (layer "F.Cu") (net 30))
 (segment (start 167.41 118.24) (end 168.73 118.24) (width 0.2) (layer "F.Cu") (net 30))
 (segment (start 142.72 129) (end 165.05 129) (width 0.2) (layer "F.Cu") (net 30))
 (segment (start 152.5 121) (end 160.95 121) (width 0.2) (layer "F.Cu") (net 24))
 (segment (start 161.75 116.8) (end 167.93 110.62) (width 0.2) (layer "F.Cu") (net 24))
 (segment (start 161.75 120.2) (end 161.75 116.8) (width 0.2) (layer "F.Cu") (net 24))
 (segment (start 160.95 121) (end 161.75 120.2) (width 0.2) (layer "F.Cu") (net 24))
 (segment (start 167.93 110.62) (end 168.73 110.62) (width 0.2) (layer "F.Cu") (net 24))
 (segment (start 161.95 123.55) (end 162.4 123.1) (width 0.2) (layer "F.Cu") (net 25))
 (segment (start 149.96 123.54) (end 158.96 123.54) (width 0.2) (layer "F.Cu") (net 25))
 (segment (start 158.97 123.55) (end 161.95 123.55) (width 0.2) (layer "F.Cu") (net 25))
 (segment (start 170.06 111.95) (end 171.27 113.16) (width 0.2) (layer "F.Cu") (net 25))
 (segment (start 168 111.95) (end 170.06 111.95) (width 0.2) (layer "F.Cu") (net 25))
 (segment (start 162.4 117.55) (end 168 111.95) (width 0.2) (layer "F.Cu") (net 25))
 (segment (start 158.96 123.54) (end 158.97 123.55) (width 0.2) (layer "F.Cu") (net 25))
 (segment (start 162.4 123.1) (end 162.4 117.55) (width 0.2) (layer "F.Cu") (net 25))
 (segment (start 170.05 104.32) (end 171.27 105.54) (width 0.2) (layer "F.Cu") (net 19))
 (segment (start 152.5 108.3) (end 163.45 108.3) (width 0.2) (layer "F.Cu") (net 19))
 (segment (start 167.45 104.3) (end 170.05 104.3) (width 0.2) (layer "F.Cu") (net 19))
 (segment (start 170.05 104.3) (end 170.05 104.32) (width 0.2) (layer "F.Cu") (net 19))
 (segment (start 163.45 108.3) (end 167.45 104.3) (width 0.2) (layer "F.Cu") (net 19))
 (segment (start 120.18 101.02) (end 120.15 101.05) (width 0.2) (layer "F.Cu") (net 35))
 (segment (start 120.15 101.05) (end 122.32 103.22) (width 1) (layer "F.Cu") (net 35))
 (segment (start 122.32 103.22) (end 124.56 103.22) (width 1) (layer "F.Cu") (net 35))
 (segment (start 112.08 101.02) (end 120.18 101.02) (width 1) (layer "F.Cu") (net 35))
 (segment (start 112.42 110.84) (end 112.08 111.18) (width 0.2) (layer "F.Cu") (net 39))
 (segment (start 124.56 110.84) (end 112.42 110.84) (width 0.2) (layer "F.Cu") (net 39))
 (segment (start 112.42 108.3) (end 112.08 108.64) (width 0.2) (layer "F.Cu") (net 38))
 (segment (start 124.56 108.3) (end 112.42 108.3) (width 0.2) (layer "F.Cu") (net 38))
 (segment (start 109.86 103.56) (end 108.45 102.15) (width 1) (layer "F.Cu") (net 36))
 (segment (start 108.45 102.15) (end 108.45 99.95) (width 1) (layer "F.Cu") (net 36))
 (segment (start 108.45 99.95) (end 110.26 98.14) (width 1) (layer "F.Cu") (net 36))
 (segment (start 112.08 103.56) (end 109.86 103.56) (width 1) (layer "F.Cu") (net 36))
 (segment (start 110.26 98.14) (end 124.56 98.14) (width 1) (layer "F.Cu") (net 36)))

